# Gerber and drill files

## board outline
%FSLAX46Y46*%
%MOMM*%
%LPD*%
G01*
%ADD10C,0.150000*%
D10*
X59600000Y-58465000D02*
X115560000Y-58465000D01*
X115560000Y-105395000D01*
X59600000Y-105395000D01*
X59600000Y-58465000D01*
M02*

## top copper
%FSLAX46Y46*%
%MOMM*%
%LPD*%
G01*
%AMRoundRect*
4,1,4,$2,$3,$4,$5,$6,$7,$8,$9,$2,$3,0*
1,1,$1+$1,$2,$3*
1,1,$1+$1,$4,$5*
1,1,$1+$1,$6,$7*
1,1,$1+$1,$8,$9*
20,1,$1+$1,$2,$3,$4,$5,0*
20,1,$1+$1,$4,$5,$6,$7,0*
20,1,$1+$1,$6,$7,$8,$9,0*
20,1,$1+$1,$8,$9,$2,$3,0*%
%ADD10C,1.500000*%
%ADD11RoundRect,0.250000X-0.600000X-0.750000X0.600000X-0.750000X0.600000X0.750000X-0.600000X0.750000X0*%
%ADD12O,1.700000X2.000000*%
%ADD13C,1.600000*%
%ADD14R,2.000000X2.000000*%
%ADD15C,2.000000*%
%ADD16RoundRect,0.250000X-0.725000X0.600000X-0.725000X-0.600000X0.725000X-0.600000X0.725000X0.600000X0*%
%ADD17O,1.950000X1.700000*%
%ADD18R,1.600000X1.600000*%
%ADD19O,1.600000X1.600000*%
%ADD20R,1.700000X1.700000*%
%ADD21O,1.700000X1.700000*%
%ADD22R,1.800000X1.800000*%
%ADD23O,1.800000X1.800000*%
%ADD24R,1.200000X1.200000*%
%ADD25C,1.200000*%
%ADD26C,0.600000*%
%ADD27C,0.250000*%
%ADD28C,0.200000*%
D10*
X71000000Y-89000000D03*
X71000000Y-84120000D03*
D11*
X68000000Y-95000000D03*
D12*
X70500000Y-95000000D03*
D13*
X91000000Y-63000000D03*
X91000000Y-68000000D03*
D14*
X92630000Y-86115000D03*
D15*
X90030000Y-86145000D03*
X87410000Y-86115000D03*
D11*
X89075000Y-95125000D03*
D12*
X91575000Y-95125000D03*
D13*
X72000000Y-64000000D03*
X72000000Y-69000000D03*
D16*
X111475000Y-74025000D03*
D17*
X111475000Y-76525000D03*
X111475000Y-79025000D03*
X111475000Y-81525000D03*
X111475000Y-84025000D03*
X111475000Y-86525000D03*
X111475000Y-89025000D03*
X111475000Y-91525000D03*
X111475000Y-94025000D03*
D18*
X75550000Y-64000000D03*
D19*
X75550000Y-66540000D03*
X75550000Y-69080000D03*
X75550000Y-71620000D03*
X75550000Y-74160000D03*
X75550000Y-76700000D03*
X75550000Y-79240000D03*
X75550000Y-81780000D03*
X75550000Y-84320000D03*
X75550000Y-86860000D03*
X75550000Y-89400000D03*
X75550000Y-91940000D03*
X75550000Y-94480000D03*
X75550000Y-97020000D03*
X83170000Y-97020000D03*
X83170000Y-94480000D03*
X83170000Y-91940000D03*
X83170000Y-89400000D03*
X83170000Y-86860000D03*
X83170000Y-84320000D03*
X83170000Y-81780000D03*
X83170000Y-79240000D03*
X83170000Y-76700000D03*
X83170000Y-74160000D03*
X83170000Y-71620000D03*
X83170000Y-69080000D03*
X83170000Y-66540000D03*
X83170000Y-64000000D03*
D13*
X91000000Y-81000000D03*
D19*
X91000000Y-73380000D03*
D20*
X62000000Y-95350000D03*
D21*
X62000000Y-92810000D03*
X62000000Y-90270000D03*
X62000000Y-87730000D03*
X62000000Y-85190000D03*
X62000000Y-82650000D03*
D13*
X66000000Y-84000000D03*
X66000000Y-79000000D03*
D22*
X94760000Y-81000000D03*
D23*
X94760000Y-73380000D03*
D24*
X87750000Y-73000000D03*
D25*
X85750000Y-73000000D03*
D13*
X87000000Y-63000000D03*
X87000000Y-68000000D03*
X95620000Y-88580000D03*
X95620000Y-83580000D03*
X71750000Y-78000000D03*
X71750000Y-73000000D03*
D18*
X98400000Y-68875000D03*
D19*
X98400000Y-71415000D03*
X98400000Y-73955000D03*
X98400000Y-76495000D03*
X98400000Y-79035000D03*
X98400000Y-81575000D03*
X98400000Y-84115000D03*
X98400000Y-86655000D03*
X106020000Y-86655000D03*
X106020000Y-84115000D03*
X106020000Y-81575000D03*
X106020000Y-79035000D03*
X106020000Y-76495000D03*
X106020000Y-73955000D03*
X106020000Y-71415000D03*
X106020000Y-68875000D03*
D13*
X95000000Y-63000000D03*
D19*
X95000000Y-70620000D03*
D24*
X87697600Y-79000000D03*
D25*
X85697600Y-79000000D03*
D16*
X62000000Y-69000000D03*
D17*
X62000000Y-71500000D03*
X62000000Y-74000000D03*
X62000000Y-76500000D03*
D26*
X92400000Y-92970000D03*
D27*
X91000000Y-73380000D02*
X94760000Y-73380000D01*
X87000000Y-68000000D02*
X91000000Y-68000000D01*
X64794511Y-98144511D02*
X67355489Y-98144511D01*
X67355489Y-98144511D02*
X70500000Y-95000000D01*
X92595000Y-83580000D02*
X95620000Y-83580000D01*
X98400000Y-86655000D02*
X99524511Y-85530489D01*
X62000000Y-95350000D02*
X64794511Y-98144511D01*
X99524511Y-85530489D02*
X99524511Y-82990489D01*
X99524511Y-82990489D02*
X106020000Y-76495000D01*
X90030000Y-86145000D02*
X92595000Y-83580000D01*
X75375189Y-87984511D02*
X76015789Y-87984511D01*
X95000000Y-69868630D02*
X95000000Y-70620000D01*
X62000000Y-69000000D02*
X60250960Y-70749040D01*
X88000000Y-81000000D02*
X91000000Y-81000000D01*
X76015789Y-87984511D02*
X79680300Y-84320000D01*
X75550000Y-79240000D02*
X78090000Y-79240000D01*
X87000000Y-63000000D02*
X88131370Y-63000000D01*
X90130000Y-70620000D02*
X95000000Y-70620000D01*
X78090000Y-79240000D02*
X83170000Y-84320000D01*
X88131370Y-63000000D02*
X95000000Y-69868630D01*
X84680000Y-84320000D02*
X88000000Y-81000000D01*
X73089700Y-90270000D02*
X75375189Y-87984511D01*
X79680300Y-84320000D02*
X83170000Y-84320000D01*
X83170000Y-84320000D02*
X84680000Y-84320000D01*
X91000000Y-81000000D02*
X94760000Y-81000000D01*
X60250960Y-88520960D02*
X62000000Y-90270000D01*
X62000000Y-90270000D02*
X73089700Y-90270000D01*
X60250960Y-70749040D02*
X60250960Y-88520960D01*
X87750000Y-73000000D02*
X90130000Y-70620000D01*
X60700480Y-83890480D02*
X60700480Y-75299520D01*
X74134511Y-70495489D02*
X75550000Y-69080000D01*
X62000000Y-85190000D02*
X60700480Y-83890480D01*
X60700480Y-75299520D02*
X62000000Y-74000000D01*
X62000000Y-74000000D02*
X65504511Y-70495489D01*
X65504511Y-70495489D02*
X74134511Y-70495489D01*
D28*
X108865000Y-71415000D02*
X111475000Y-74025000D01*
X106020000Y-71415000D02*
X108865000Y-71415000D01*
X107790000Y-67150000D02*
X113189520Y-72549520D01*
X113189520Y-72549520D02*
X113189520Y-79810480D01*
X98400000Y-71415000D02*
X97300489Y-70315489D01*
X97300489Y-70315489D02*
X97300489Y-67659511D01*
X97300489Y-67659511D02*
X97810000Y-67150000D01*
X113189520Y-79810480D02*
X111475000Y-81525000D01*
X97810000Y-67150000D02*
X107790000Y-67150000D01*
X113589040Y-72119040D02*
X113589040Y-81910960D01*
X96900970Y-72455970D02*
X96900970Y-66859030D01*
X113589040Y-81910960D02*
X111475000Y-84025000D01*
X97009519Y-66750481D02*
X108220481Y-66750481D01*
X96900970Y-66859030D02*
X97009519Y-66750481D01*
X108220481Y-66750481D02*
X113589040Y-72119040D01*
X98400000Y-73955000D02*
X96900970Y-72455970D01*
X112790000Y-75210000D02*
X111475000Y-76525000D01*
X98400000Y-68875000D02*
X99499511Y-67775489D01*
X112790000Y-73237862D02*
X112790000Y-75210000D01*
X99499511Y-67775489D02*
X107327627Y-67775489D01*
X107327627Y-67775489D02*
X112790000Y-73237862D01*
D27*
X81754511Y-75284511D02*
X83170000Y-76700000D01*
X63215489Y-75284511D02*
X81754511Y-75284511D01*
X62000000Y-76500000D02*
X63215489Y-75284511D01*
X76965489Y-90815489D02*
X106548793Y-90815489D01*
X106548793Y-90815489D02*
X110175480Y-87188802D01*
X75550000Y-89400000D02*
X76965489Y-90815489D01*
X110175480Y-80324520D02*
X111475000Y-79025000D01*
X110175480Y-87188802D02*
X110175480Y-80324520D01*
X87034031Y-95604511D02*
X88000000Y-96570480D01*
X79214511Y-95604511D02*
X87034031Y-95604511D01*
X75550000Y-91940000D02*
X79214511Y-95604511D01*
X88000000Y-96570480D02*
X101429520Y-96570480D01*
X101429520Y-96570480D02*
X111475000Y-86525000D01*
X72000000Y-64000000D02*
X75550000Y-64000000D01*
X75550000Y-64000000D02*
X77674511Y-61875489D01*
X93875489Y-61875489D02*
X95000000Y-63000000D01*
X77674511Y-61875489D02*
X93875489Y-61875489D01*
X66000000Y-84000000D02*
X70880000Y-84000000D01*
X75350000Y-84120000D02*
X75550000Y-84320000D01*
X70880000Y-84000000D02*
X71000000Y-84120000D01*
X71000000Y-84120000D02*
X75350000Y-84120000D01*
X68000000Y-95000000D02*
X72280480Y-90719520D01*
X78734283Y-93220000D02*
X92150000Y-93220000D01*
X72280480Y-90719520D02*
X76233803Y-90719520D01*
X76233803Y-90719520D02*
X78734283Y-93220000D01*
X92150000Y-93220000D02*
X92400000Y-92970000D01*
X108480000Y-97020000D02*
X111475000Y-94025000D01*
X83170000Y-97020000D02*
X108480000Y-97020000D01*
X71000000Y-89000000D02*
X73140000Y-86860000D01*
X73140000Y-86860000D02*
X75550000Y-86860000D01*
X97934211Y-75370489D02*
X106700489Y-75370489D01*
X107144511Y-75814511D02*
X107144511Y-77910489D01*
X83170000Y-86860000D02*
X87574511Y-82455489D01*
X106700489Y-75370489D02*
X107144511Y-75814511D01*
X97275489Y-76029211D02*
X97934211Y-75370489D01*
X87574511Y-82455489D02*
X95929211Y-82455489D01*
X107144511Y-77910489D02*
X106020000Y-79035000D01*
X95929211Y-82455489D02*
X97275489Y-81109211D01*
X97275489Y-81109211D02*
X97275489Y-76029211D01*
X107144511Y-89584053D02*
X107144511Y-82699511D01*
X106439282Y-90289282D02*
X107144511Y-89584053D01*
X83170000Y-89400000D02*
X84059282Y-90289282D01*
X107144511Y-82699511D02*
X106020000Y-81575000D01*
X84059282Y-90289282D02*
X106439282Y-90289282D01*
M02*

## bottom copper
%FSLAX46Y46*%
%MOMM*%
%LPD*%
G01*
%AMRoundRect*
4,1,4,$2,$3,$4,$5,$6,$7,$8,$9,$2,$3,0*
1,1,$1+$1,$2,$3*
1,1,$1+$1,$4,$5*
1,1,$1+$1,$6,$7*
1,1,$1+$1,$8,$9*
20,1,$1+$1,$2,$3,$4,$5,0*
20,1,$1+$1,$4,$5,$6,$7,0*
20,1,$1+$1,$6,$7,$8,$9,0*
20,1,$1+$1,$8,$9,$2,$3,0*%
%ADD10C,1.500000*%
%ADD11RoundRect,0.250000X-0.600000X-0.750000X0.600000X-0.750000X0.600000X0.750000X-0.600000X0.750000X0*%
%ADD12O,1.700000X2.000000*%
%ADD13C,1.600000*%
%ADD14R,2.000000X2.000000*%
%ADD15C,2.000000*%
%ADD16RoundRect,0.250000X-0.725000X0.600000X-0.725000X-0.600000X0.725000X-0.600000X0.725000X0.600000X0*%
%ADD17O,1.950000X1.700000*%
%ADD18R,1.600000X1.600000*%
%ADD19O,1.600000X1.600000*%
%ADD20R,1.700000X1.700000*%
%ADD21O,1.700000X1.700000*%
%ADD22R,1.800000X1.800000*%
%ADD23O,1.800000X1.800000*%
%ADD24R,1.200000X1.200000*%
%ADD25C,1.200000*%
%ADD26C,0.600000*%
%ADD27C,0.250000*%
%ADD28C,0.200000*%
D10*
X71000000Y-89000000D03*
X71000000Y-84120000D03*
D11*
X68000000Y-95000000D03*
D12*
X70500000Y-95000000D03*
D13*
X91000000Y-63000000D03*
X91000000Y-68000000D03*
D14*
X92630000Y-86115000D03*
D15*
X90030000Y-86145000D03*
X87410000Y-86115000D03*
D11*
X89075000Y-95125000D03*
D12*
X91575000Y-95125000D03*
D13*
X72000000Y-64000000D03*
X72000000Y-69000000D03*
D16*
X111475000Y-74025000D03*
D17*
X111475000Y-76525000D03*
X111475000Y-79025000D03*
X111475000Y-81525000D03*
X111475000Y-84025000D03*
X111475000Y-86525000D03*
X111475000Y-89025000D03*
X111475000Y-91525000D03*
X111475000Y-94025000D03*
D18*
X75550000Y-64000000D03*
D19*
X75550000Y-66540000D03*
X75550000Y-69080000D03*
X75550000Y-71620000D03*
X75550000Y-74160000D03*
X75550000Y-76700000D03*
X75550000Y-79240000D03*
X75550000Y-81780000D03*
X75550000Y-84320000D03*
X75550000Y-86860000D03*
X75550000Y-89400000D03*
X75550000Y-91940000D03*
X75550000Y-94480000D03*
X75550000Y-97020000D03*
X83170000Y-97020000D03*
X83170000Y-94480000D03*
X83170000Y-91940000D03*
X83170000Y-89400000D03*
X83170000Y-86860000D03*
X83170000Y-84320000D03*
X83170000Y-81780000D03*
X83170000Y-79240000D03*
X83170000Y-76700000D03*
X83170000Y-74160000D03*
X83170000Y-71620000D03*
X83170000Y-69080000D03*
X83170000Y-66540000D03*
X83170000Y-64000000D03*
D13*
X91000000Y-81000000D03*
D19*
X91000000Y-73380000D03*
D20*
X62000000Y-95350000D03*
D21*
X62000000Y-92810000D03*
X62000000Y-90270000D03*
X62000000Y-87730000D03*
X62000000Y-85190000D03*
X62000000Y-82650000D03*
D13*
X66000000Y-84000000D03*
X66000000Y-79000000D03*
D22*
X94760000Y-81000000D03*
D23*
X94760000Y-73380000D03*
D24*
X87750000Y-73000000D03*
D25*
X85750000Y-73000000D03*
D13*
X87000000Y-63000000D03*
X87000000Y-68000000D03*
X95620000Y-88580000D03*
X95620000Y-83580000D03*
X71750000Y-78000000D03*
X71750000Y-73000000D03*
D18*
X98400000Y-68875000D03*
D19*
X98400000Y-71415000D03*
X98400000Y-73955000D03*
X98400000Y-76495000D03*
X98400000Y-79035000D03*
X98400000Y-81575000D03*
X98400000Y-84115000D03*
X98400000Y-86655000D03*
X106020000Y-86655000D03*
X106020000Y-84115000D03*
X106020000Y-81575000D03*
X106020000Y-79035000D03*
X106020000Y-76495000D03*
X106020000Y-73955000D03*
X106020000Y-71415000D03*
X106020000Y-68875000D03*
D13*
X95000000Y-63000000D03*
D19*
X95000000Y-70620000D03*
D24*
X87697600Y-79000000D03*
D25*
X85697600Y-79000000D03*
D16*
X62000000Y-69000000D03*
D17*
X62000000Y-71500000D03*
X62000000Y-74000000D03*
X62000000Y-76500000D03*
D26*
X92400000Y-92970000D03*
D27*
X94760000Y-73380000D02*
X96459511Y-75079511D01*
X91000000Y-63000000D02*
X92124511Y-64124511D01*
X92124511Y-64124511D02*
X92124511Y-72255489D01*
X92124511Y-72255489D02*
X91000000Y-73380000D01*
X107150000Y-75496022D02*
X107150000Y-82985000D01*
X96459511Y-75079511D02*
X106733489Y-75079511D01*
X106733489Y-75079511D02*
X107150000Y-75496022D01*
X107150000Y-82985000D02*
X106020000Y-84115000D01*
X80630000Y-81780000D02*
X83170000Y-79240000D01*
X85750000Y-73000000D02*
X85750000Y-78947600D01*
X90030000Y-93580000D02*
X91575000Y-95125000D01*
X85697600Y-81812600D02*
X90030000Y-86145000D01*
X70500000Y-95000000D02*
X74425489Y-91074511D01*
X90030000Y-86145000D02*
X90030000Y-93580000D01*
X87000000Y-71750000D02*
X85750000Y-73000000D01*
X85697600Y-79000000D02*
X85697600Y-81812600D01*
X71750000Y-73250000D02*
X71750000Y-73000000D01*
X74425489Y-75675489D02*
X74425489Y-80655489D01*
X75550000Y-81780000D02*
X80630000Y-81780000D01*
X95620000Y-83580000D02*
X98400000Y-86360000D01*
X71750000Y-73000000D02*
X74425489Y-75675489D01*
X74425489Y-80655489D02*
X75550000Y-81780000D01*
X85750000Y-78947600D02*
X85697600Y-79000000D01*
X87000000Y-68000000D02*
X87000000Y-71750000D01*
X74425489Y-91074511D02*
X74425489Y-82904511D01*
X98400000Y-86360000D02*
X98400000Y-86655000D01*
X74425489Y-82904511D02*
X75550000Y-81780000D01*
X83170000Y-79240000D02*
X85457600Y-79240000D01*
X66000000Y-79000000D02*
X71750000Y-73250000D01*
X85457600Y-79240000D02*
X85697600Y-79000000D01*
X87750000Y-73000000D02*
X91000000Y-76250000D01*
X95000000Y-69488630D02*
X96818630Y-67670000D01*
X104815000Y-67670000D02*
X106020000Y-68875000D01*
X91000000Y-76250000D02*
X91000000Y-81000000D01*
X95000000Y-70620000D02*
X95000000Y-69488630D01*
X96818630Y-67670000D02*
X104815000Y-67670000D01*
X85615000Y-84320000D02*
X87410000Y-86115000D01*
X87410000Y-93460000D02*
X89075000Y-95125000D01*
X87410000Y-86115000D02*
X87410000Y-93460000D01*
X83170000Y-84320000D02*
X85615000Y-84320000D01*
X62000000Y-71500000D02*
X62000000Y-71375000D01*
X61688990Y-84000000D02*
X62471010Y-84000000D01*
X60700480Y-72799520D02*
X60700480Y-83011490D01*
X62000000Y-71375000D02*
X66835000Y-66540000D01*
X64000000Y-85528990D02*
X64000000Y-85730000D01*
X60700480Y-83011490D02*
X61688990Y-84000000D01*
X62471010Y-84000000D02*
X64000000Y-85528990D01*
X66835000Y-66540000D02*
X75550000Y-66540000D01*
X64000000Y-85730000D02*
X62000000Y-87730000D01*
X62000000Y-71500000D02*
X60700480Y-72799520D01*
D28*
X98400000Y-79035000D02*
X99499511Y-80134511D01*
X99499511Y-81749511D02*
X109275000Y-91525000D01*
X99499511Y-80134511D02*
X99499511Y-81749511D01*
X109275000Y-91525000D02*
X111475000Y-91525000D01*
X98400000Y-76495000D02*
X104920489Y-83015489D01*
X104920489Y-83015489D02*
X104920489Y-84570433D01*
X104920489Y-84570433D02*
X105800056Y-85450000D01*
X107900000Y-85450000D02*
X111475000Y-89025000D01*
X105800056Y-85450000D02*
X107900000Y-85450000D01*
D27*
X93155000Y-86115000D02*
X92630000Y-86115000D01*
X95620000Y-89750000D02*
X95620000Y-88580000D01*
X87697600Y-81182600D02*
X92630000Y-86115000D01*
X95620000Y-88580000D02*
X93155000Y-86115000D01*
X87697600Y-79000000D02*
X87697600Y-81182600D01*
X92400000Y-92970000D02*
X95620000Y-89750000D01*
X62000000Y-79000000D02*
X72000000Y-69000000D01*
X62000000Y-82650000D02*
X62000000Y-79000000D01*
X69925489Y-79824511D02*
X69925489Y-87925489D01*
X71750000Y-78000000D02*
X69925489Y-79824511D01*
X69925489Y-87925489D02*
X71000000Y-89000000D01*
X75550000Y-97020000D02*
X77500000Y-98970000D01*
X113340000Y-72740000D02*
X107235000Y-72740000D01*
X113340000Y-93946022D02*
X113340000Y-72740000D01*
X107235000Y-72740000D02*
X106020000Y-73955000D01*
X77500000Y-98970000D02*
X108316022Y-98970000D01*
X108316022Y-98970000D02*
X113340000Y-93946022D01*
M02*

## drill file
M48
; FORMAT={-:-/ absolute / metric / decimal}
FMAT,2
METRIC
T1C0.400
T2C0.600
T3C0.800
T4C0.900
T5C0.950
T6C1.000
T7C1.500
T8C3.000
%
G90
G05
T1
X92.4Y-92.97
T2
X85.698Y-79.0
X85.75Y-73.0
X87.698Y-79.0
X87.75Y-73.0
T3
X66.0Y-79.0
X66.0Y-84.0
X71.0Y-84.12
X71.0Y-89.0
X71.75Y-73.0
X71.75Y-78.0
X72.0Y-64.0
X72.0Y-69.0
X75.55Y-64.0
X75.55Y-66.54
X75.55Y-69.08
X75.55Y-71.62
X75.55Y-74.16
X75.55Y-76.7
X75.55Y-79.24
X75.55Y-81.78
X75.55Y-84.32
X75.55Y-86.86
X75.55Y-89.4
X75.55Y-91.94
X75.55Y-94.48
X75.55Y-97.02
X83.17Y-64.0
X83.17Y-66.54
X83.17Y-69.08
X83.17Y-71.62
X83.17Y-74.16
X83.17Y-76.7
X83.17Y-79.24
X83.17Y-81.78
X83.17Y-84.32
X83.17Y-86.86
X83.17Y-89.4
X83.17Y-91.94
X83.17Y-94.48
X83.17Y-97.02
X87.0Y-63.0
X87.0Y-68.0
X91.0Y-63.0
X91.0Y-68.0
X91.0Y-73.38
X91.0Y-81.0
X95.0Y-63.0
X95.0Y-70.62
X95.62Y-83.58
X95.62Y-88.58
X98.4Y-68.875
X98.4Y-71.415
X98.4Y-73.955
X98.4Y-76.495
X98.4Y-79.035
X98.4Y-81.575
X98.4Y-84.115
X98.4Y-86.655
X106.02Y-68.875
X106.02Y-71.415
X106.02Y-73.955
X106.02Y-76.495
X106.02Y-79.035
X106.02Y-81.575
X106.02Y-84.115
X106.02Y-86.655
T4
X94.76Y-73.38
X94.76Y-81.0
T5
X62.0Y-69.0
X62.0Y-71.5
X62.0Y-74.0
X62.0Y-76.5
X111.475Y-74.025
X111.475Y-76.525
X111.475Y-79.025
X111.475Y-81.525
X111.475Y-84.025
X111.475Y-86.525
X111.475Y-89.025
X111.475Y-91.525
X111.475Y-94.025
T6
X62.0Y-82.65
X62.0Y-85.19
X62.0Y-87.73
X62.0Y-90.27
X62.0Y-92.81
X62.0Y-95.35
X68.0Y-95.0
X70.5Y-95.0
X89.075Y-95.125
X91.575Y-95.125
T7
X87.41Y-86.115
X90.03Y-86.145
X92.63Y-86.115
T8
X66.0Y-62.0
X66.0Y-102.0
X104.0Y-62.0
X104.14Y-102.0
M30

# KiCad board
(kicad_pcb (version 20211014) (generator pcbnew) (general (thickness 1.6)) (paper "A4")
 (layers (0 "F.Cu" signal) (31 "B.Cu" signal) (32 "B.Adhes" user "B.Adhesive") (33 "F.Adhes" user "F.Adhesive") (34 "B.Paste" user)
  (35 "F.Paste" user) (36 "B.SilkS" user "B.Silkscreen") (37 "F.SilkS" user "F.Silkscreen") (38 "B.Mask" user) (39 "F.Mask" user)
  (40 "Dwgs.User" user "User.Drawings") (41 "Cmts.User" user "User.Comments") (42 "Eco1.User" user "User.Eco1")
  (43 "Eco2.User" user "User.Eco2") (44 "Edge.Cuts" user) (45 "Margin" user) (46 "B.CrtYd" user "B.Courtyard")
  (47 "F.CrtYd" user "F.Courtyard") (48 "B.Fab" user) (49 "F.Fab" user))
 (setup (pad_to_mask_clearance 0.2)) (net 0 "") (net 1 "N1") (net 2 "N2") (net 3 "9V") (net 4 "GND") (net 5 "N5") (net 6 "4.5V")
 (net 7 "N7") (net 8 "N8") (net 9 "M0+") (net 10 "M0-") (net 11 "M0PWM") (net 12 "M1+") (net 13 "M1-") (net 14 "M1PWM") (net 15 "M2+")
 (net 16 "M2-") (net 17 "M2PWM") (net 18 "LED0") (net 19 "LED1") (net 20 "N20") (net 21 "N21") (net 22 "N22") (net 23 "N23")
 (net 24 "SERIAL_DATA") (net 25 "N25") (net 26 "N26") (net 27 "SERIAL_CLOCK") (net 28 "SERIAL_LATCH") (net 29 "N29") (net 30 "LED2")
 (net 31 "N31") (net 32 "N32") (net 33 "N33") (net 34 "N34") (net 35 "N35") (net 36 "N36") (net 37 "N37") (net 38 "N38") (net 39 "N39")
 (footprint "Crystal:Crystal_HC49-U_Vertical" (layer "F.Cu") (at 71 89 90)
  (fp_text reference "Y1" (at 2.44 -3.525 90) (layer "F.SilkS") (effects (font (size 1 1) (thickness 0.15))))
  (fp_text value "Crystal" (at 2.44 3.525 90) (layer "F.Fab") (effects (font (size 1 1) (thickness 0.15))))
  (pad "1" thru_hole circle (at 0 0 90) (size 1.5 1.5) (drill 0.8) (layers *.Cu *.Mask) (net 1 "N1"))
  (pad "2" thru_hole circle (at 4.88 0 90) (size 1.5 1.5) (drill 0.8) (layers *.Cu *.Mask) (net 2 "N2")))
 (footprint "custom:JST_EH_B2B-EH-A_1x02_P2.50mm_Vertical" (layer "F.Cu") (at 68 95)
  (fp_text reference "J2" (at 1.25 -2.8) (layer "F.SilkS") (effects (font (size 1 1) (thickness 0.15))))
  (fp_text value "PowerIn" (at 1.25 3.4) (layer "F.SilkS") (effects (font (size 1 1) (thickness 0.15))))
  (pad "1" thru_hole roundrect locked (at 0 0) (size 1.7 2) (drill 1) (layers *.Cu *.Mask) (roundrect_rratio 0.147059) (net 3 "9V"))
  (pad "2" thru_hole oval locked (at 2.5 0) (size 1.7 2) (drill 1) (layers *.Cu *.Mask) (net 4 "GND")))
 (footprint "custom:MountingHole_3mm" (layer "F.Cu") (at 104.14 102)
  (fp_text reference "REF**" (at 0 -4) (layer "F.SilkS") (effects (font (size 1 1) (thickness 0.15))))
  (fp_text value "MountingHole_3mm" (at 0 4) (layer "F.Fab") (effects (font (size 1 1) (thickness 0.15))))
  (pad "" np_thru_hole circle locked (at 0 0) (size 3 3) (drill 3) (layers *.Cu *.Mask)))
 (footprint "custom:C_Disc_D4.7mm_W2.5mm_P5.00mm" (layer "F.Cu") (at 91 63 -90)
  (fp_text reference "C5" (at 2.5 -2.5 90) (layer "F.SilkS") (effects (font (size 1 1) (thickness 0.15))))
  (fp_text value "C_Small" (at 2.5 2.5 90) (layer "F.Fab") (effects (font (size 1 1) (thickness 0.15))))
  (pad "1" thru_hole circle locked (at 0 0 270) (size 1.6 1.6) (drill 0.8) (layers *.Cu *.Mask) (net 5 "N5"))
  (pad "2" thru_hole circle locked (at 5 0 270) (size 1.6 1.6) (drill 0.8) (layers *.Cu *.Mask) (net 4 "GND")))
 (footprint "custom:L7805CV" (layer "F.Cu") (at 93.64 87.035 180)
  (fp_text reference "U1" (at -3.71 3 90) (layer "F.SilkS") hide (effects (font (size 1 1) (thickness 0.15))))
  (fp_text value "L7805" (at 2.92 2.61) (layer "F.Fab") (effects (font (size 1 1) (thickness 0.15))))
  (pad "1" thru_hole rect (at 1.01 0.92 180) (size 2 2) (drill 1.5) (layers *.Cu *.Mask) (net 3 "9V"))
  (pad "2" thru_hole circle (at 3.61 0.89 180) (size 2 2) (drill 1.5) (layers *.Cu *.Mask) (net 4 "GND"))
  (pad "3" thru_hole circle (at 6.23 0.92 180) (size 2 2) (drill 1.5) (layers *.Cu *.Mask) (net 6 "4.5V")))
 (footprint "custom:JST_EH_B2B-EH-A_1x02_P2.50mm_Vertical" (layer "F.Cu") (at 89.075 95.125)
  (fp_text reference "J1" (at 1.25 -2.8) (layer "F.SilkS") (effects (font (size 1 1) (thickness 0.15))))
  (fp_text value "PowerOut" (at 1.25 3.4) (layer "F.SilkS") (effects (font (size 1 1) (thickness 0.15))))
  (pad "1" thru_hole roundrect locked (at 0 0) (size 1.7 2) (drill 1) (layers *.Cu *.Mask) (roundrect_rratio 0.147059) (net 6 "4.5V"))
  (pad "2" thru_hole oval locked (at 2.5 0) (size 1.7 2) (drill 1) (layers *.Cu *.Mask) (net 4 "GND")))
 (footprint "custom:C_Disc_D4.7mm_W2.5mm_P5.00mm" (layer "F.Cu") (at 72 64 -90)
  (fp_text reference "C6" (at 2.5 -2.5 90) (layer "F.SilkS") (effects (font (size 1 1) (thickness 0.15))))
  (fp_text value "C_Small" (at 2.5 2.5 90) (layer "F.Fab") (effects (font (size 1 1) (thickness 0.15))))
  (pad "1" thru_hole circle locked (at 0 0 270) (size 1.6 1.6) (drill 0.8) (layers *.Cu *.Mask) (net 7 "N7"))
  (pad "2" thru_hole circle locked (at 5 0 270) (size 1.6 1.6) (drill 0.8) (layers *.Cu *.Mask) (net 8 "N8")))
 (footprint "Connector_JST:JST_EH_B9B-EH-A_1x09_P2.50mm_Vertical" (layer "F.Cu") (at 111.475 74.025 -90)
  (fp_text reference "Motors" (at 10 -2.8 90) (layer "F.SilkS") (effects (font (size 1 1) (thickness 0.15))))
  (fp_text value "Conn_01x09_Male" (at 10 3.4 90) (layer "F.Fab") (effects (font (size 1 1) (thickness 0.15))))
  (pad "1" thru_hole roundrect (at 0 0 270) (size 1.7 1.95) (drill 0.95) (layers *.Cu *.Mask) (roundrect_rratio 0.147059) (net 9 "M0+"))
  (pad "2" thru_hole oval (at 2.5 0 270) (size 1.7 1.95) (drill 0.95) (layers *.Cu *.Mask) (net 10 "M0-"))
  (pad "3" thru_hole oval (at 5 0 270) (size 1.7 1.95) (drill 0.95) (layers *.Cu *.Mask) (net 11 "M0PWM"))
  (pad "4" thru_hole oval (at 7.5 0 270) (size 1.7 1.95) (drill 0.95) (layers *.Cu *.Mask) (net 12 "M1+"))
  (pad "5" thru_hole oval (at 10 0 270) (size 1.7 1.95) (drill 0.95) (layers *.Cu *.Mask) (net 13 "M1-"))
  (pad "6" thru_hole oval (at 12.5 0 270) (size 1.7 1.95) (drill 0.95) (layers *.Cu *.Mask) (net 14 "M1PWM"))
  (pad "7" thru_hole oval (at 15 0 270) (size 1.7 1.95) (drill 0.95) (layers *.Cu *.Mask) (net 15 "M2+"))
  (pad "8" thru_hole oval (at 17.5 0 270) (size 1.7 1.95) (drill 0.95) (layers *.Cu *.Mask) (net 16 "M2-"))
  (pad "9" thru_hole oval (at 20 0 270) (size 1.7 1.95) (drill 0.95) (layers *.Cu *.Mask) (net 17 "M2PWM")))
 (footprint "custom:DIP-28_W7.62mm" (layer "F.Cu") (at 75.55 64)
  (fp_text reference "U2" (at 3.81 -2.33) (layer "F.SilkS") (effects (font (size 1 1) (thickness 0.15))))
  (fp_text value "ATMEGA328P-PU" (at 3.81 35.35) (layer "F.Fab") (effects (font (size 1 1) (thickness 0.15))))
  (pad "1" thru_hole rect locked (at 0 0) (size 1.6 1.6) (drill 0.8) (layers *.Cu *.Mask) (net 7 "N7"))
  (pad "2" thru_hole oval locked (at 0 2.54) (size 1.6 1.6) (drill 0.8) (layers *.Cu *.Mask) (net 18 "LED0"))
  (pad "3" thru_hole oval locked (at 0 5.08) (size 1.6 1.6) (drill 0.8) (layers *.Cu *.Mask) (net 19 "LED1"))
  (pad "4" thru_hole oval locked (at 0 7.62) (size 1.6 1.6) (drill 0.8) (layers *.Cu *.Mask) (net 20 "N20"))
  (pad "5" thru_hole oval locked (at 0 10.16) (size 1.6 1.6) (drill 0.8) (layers *.Cu *.Mask) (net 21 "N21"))
  (pad "6" thru_hole oval locked (at 0 12.7) (size 1.6 1.6) (drill 0.8) (layers *.Cu *.Mask) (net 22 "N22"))
  (pad "7" thru_hole oval locked (at 0 15.24) (size 1.6 1.6) (drill 0.8) (layers *.Cu *.Mask) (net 6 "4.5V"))
  (pad "8" thru_hole oval locked (at 0 17.78) (size 1.6 1.6) (drill 0.8) (layers *.Cu *.Mask) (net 4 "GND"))
  (pad "9" thru_hole oval locked (at 0 20.32) (size 1.6 1.6) (drill 0.8) (layers *.Cu *.Mask) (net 2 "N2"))
  (pad "10" thru_hole oval locked (at 0 22.86) (size 1.6 1.6) (drill 0.8) (layers *.Cu *.Mask) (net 1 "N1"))
  (pad "11" thru_hole oval locked (at 0 25.4) (size 1.6 1.6) (drill 0.8) (layers *.Cu *.Mask) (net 11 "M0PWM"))
  (pad "12" thru_hole oval locked (at 0 27.94) (size 1.6 1.6) (drill 0.8) (layers *.Cu *.Mask) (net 14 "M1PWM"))
  (pad "13" thru_hole oval locked (at 0 30.48) (size 1.6 1.6) (drill 0.8) (layers *.Cu *.Mask) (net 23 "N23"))
  (pad "14" thru_hole oval locked (at 0 33.02) (size 1.6 1.6) (drill 0.8) (layers *.Cu *.Mask) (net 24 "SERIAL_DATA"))
  (pad "15" thru_hole oval locked (at 7.62 33.02) (size 1.6 1.6) (drill 0.8) (layers *.Cu *.Mask) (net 17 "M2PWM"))
  (pad "16" thru_hole oval locked (at 7.62 30.48) (size 1.6 1.6) (drill 0.8) (layers *.Cu *.Mask) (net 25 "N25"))
  (pad "17" thru_hole oval locked (at 7.62 27.94) (size 1.6 1.6) (drill 0.8) (layers *.Cu *.Mask) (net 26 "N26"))
  (pad "18" thru_hole oval locked (at 7.62 25.4) (size 1.6 1.6) (drill 0.8) (layers *.Cu *.Mask) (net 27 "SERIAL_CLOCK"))
  (pad "19" thru_hole oval locked (at 7.62 22.86) (size 1.6 1.6) (drill 0.8) (layers *.Cu *.Mask) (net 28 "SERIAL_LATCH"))
  (pad "20" thru_hole oval locked (at 7.62 20.32) (size 1.6 1.6) (drill 0.8) (layers *.Cu *.Mask) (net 6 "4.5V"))
  (pad "21" thru_hole oval locked (at 7.62 17.78) (size 1.6 1.6) (drill 0.8) (layers *.Cu *.Mask) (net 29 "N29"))
  (pad "22" thru_hole oval locked (at 7.62 15.24) (size 1.6 1.6) (drill 0.8) (layers *.Cu *.Mask) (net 4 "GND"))
  (pad "23" thru_hole oval locked (at 7.62 12.7) (size 1.6 1.6) (drill 0.8) (layers *.Cu *.Mask) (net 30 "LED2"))
  (pad "24" thru_hole oval locked (at 7.62 10.16) (size 1.6 1.6) (drill 0.8) (layers *.Cu *.Mask) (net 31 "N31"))
  (pad "25" thru_hole oval locked (at 7.62 7.62) (size 1.6 1.6) (drill 0.8) (layers *.Cu *.Mask) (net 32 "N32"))
  (pad "26" thru_hole oval locked (at 7.62 5.08) (size 1.6 1.6) (drill 0.8) (layers *.Cu *.Mask) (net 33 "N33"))
  (pad "27" thru_hole oval locked (at 7.62 2.54) (size 1.6 1.6) (drill 0.8) (layers *.Cu *.Mask) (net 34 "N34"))
  (pad "28" thru_hole oval locked (at 7.62 0) (size 1.6 1.6) (drill 0.8) (layers *.Cu *.Mask) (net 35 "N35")))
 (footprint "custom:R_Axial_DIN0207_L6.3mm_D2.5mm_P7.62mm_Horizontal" (layer "F.Cu") (at 91 81 90)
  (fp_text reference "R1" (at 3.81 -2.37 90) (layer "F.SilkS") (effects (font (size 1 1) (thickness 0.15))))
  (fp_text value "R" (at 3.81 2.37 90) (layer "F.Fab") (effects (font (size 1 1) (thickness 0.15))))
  (pad "1" thru_hole circle locked (at 0 0 90) (size 1.6 1.6) (drill 0.8) (layers *.Cu *.Mask) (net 6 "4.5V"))
  (pad "2" thru_hole oval locked (at 7.62 0 90) (size 1.6 1.6) (drill 0.8) (layers *.Cu *.Mask) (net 5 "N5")))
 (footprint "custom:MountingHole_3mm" (layer "F.Cu") (at 104 62)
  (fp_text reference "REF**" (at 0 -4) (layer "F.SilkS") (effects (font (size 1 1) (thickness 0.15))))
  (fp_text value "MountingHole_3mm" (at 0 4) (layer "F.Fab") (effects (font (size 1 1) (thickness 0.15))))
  (pad "" np_thru_hole circle locked (at 0 0) (size 3 3) (drill 3) (layers F&B.Cu *.Mask)))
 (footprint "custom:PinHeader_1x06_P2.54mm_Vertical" (layer "F.Cu") (at 62 95.35 180)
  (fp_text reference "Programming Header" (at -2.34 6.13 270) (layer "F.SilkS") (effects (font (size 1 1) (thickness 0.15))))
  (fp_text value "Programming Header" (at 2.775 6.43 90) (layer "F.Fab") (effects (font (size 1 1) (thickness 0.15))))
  (pad "1" thru_hole rect locked (at 0 0 180) (size 1.7 1.7) (drill 1) (layers *.Cu *.Mask) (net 4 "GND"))
  (pad "2" thru_hole oval locked (at 0 2.54 180) (size 1.7 1.7) (drill 1) (layers *.Cu *.Mask) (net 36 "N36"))
  (pad "3" thru_hole oval locked (at 0 5.08 180) (size 1.7 1.7) (drill 1) (layers *.Cu *.Mask) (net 6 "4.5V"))
  (pad "4" thru_hole oval locked (at 0 7.62 180) (size 1.7 1.7) (drill 1) (layers *.Cu *.Mask) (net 18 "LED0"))
  (pad "5" thru_hole oval locked (at 0 10.16 180) (size 1.7 1.7) (drill 1) (layers *.Cu *.Mask) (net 19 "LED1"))
  (pad "6" thru_hole oval locked (at 0 12.7 180) (size 1.7 1.7) (drill 1) (layers *.Cu *.Mask) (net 8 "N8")))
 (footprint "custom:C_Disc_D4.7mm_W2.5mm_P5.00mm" (layer "F.Cu") (at 66 84 90)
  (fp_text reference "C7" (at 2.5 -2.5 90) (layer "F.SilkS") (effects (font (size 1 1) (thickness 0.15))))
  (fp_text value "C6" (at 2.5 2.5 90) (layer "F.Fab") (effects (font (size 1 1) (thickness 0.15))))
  (pad "1" thru_hole circle locked (at 0 0 90) (size 1.6 1.6) (drill 0.8) (layers *.Cu *.Mask) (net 2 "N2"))
  (pad "2" thru_hole circle locked (at 5 0 90) (size 1.6 1.6) (drill 0.8) (layers *.Cu *.Mask) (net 4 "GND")))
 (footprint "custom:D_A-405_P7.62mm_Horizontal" (layer "F.Cu") (at 94.76 81 90)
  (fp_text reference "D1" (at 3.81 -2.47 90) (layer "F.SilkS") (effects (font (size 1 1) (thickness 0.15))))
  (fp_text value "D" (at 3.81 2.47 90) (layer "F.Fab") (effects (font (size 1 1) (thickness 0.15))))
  (pad "1" thru_hole rect locked (at 0 0 90) (size 1.8 1.8) (drill 0.9) (layers *.Cu *.Mask) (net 6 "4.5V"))
  (pad "2" thru_hole oval locked (at 7.62 0 90) (size 1.8 1.8) (drill 0.9) (layers *.Cu *.Mask) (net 5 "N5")))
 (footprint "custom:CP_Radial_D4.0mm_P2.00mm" (layer "F.Cu") (at 87.75 73 180)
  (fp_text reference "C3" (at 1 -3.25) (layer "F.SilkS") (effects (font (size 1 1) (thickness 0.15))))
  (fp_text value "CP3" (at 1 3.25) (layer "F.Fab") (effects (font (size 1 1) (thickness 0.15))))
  (pad "1" thru_hole rect locked (at 0 0 180) (size 1.2 1.2) (drill 0.6) (layers *.Cu *.Mask) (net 6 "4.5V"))
  (pad "2" thru_hole circle locked (at 2 0 180) (size 1.2 1.2) (drill 0.6) (layers *.Cu *.Mask) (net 4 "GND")))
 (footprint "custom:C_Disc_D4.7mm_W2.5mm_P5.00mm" (layer "F.Cu") (at 87 63 -90)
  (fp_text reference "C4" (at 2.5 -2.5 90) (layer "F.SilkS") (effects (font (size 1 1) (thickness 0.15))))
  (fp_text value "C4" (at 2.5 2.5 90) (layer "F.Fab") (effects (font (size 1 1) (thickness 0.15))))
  (pad "1" thru_hole circle locked (at 0 0 270) (size 1.6 1.6) (drill 0.8) (layers *.Cu *.Mask) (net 6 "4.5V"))
  (pad "2" thru_hole circle locked (at 5 0 270) (size 1.6 1.6) (drill 0.8) (layers *.Cu *.Mask) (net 4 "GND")))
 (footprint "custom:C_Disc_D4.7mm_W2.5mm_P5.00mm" (layer "F.Cu") (at 95.62 88.58 90)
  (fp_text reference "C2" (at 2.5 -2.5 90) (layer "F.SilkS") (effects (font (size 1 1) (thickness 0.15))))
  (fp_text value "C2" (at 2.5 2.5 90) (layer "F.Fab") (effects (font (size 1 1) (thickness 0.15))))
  (pad "1" thru_hole circle locked (at 0 0 90) (size 1.6 1.6) (drill 0.8) (layers *.Cu *.Mask) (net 3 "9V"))
  (pad "2" thru_hole circle locked (at 5 0 90) (size 1.6 1.6) (drill 0.8) (layers *.Cu *.Mask) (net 4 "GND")))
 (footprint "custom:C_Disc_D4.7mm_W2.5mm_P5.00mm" (layer "F.Cu") (at 71.75 78 90)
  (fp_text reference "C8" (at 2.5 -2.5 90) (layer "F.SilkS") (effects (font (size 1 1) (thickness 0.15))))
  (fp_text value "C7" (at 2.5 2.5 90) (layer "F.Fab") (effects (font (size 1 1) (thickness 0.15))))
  (pad "1" thru_hole circle locked (at 0 0 90) (size 1.6 1.6) (drill 0.8) (layers *.Cu *.Mask) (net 1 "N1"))
  (pad "2" thru_hole circle locked (at 5 0 90) (size 1.6 1.6) (drill 0.8) (layers *.Cu *.Mask) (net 4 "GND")))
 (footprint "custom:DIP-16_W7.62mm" (layer "F.Cu") (at 98.4 68.875)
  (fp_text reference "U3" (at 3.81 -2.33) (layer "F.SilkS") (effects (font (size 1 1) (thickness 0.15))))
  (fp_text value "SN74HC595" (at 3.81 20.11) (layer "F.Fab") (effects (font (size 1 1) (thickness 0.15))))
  (pad "1" thru_hole rect locked (at 0 0) (size 1.6 1.6) (drill 0.8) (layers *.Cu *.Mask) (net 10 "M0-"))
  (pad "2" thru_hole oval locked (at 0 2.54) (size 1.6 1.6) (drill 0.8) (layers *.Cu *.Mask) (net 12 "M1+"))
  (pad "3" thru_hole oval locked (at 0 5.08) (size 1.6 1.6) (drill 0.8) (layers *.Cu *.Mask) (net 13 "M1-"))
  (pad "4" thru_hole oval locked (at 0 7.62) (size 1.6 1.6) (drill 0.8) (layers *.Cu *.Mask) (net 15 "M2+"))
  (pad "5" thru_hole oval locked (at 0 10.16) (size 1.6 1.6) (drill 0.8) (layers *.Cu *.Mask) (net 16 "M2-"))
  (pad "6" thru_hole oval locked (at 0 12.7) (size 1.6 1.6) (drill 0.8) (layers *.Cu *.Mask) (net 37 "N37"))
  (pad "7" thru_hole oval locked (at 0 15.24) (size 1.6 1.6) (drill 0.8) (layers *.Cu *.Mask) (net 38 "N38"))
  (pad "8" thru_hole oval locked (at 0 17.78) (size 1.6 1.6) (drill 0.8) (layers *.Cu *.Mask) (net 4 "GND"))
  (pad "9" thru_hole oval locked (at 7.62 17.78) (size 1.6 1.6) (drill 0.8) (layers *.Cu *.Mask) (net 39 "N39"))
  (pad "10" thru_hole oval locked (at 7.62 15.24) (size 1.6 1.6) (drill 0.8) (layers *.Cu *.Mask) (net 5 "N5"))
  (pad "11" thru_hole oval locked (at 7.62 12.7) (size 1.6 1.6) (drill 0.8) (layers *.Cu *.Mask) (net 27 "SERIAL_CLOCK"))
  (pad "12" thru_hole oval locked (at 7.62 10.16) (size 1.6 1.6) (drill 0.8) (layers *.Cu *.Mask) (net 28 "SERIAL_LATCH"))
  (pad "13" thru_hole oval locked (at 7.62 7.62) (size 1.6 1.6) (drill 0.8) (layers *.Cu *.Mask) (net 4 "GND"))
  (pad "14" thru_hole oval locked (at 7.62 5.08) (size 1.6 1.6) (drill 0.8) (layers *.Cu *.Mask) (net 24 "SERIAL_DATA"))
  (pad "15" thru_hole oval locked (at 7.62 2.54) (size 1.6 1.6) (drill 0.8) (layers *.Cu *.Mask) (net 9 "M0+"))
  (pad "16" thru_hole oval locked (at 7.62 0) (size 1.6 1.6) (drill 0.8) (layers *.Cu *.Mask) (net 6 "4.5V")))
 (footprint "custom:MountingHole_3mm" (layer "F.Cu") (at 66 62)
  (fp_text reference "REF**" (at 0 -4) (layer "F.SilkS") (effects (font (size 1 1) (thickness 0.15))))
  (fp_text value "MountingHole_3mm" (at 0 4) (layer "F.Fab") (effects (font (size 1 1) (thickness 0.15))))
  (pad "" np_thru_hole circle locked (at 0 0) (size 3 3) (drill 3) (layers *.Cu *.Mask)))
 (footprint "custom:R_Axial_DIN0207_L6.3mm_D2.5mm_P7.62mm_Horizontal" (layer "F.Cu") (at 95 63 -90)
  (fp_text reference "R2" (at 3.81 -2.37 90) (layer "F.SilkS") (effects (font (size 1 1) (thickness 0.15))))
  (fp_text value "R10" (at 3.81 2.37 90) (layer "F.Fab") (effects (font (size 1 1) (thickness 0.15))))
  (pad "1" thru_hole circle locked (at 0 0 270) (size 1.6 1.6) (drill 0.8) (layers *.Cu *.Mask) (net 7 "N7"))
  (pad "2" thru_hole oval locked (at 7.62 0 270) (size 1.6 1.6) (drill 0.8) (layers *.Cu *.Mask) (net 6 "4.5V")))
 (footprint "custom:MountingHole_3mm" (layer "F.Cu") (at 66 102)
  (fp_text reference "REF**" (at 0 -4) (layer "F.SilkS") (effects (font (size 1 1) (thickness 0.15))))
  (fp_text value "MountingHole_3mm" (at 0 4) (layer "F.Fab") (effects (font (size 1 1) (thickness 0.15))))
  (pad "" np_thru_hole circle locked (at 0 0) (size 3 3) (drill 3) (layers *.Cu *.Mask)))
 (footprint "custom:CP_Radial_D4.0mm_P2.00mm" (layer "F.Cu") (at 87.6976 79 180)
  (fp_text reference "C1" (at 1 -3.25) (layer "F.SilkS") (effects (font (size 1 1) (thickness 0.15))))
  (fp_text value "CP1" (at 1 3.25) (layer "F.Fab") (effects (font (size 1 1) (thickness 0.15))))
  (pad "1" thru_hole rect locked (at 0 0 180) (size 1.2 1.2) (drill 0.6) (layers *.Cu *.Mask) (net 3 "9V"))
  (pad "2" thru_hole circle locked (at 2 0 180) (size 1.2 1.2) (drill 0.6) (layers *.Cu *.Mask) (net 4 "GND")))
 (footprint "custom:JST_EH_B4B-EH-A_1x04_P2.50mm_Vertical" (layer "F.Cu") (at 62 69 -90)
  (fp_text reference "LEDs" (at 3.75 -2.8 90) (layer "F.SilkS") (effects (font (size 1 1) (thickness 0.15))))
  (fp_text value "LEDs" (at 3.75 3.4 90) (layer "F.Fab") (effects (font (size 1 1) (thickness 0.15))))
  (pad "1" thru_hole roundrect locked (at 0 0 270) (size 1.7 1.95) (drill 0.95) (layers *.Cu *.Mask) (roundrect_rratio 0.147059)
   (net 6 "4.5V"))
  (pad "2" thru_hole oval locked (at 2.5 0 270) (size 1.7 1.95) (drill 0.95) (layers *.Cu *.Mask) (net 18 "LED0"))
  (pad "3" thru_hole oval locked (at 5 0 270) (size 1.7 1.95) (drill 0.95) (layers *.Cu *.Mask) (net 19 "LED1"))
  (pad "4" thru_hole oval locked (at 7.5 0 270) (size 1.7 1.95) (drill 0.95) (layers *.Cu *.Mask) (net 30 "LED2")))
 (gr_rect (start 59.6 58.465) (end 115.56 105.395) (layer "Edge.Cuts") (width 0.15) (fill none))
 (segment (start 91 73.38) (end 94.76 73.38) (width 0.25) (layer "F.Cu") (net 5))
 (segment (start 94.76 73.38) (end 96.459511 75.079511) (width 0.25) (layer "B.Cu") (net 5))
 (segment (start 91 63) (end 92.124511 64.124511) (width 0.25) (layer "B.Cu") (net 5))
 (segment (start 92.124511 64.124511) (end 92.124511 72.255489) (width 0.25) (layer "B.Cu") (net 5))
 (segment (start 92.124511 72.255489) (end 91 73.38) (width 0.25) (layer "B.Cu") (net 5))
 (segment (start 107.15 75.496022) (end 107.15 82.985) (width 0.25) (layer "B.Cu") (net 5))
 (segment (start 96.459511 75.079511) (end 106.733489 75.079511) (width 0.25) (layer "B.Cu") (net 5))
 (segment (start 106.733489 75.079511) (end 107.15 75.496022) (width 0.25) (layer "B.Cu") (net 5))
 (segment (start 107.15 82.985) (end 106.02 84.115) (width 0.25) (layer "B.Cu") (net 5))
 (segment (start 87 68) (end 91 68) (width 0.25) (layer "F.Cu") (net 4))
 (segment (start 64.794511 98.144511) (end 67.355489 98.144511) (width 0.25) (layer "F.Cu") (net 4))
 (segment (start 67.355489 98.144511) (end 70.5 95) (width 0.25) (layer "F.Cu") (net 4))
 (segment (start 92.595 83.58) (end 95.62 83.58) (width 0.25) (layer "F.Cu") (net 4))
 (segment (start 98.4 86.655) (end 99.524511 85.530489) (width 0.25) (layer "F.Cu") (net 4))
 (segment (start 62 95.35) (end 64.794511 98.144511) (width 0.25) (layer "F.Cu") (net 4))
 (segment (start 99.524511 85.530489) (end 99.524511 82.990489) (width 0.25) (layer "F.Cu") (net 4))
 (segment (start 99.524511 82.990489) (end 106.02 76.495) (width 0.25) (layer "F.Cu") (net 4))
 (segment (start 90.03 86.145) (end 92.595 83.58) (width 0.25) (layer "F.Cu") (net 4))
 (segment (start 80.63 81.78) (end 83.17 79.24) (width 0.25) (layer "B.Cu") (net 4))
 (segment (start 85.75 73) (end 85.75 78.9476) (width 0.25) (layer "B.Cu") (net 4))
 (segment (start 90.03 93.58) (end 91.575 95.125) (width 0.25) (layer "B.Cu") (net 4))
 (segment (start 85.6976 81.8126) (end 90.03 86.145) (width 0.25) (layer "B.Cu") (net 4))
 (segment (start 70.5 95) (end 74.425489 91.074511) (width 0.25) (layer "B.Cu") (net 4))
 (segment (start 90.03 86.145) (end 90.03 93.58) (width 0.25) (layer "B.Cu") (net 4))
 (segment (start 87 71.75) (end 85.75 73) (width 0.25) (layer "B.Cu") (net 4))
 (segment (start 85.6976 79) (end 85.6976 81.8126) (width 0.25) (layer "B.Cu") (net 4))
 (segment (start 71.75 73.25) (end 71.75 73) (width 0.25) (layer "B.Cu") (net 4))
 (segment (start 74.425489 75.675489) (end 74.425489 80.655489) (width 0.25) (layer "B.Cu") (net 4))
 (segment (start 75.55 81.78) (end 80.63 81.78) (width 0.25) (layer "B.Cu") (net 4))
 (segment (start 95.62 83.58) (end 98.4 86.36) (width 0.25) (layer "B.Cu") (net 4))
 (segment (start 71.75 73) (end 74.425489 75.675489) (width 0.25) (layer "B.Cu") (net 4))
 (segment (start 74.425489 80.655489) (end 75.55 81.78) (width 0.25) (layer "B.Cu") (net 4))
 (segment (start 85.75 78.9476) (end 85.6976 79) (width 0.25) (layer "B.Cu") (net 4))
 (segment (start 87 68) (end 87 71.75) (width 0.25) (layer "B.Cu") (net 4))
 (segment (start 74.425489 91.074511) (end 74.425489 82.904511) (width 0.25) (layer "B.Cu") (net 4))
 (segment (start 98.4 86.36) (end 98.4 86.655) (width 0.25) (layer "B.Cu") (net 4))
 (segment (start 74.425489 82.904511) (end 75.55 81.78) (width 0.25) (layer "B.Cu") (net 4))
 (segment (start 83.17 79.24) (end 85.4576 79.24) (width 0.25) (layer "B.Cu") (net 4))
 (segment (start 66 79) (end 71.75 73.25) (width 0.25) (layer "B.Cu") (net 4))
 (segment (start 85.4576 79.24) (end 85.6976 79) (width 0.25) (layer "B.Cu") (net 4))
 (segment (start 75.375189 87.984511) (end 76.015789 87.984511) (width 0.25) (layer "F.Cu") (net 6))
 (segment (start 95 69.86863) (end 95 70.62) (width 0.25) (layer "F.Cu") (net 6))
 (segment (start 62 69) (end 60.25096 70.74904) (width 0.25) (layer "F.Cu") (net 6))
 (segment (start 88 81) (end 91 81) (width 0.25) (layer "F.Cu") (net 6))
 (segment (start 76.015789 87.984511) (end 79.6803 84.32) (width 0.25) (layer "F.Cu") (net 6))
 (segment (start 75.55 79.24) (end 78.09 79.24) (width 0.25) (layer "F.Cu") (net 6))
 (segment (start 87 63) (end 88.13137 63) (width 0.25) (layer "F.Cu") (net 6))
 (segment (start 90.13 70.62) (end 95 70.62) (width 0.25) (layer "F.Cu") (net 6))
 (segment (start 78.09 79.24) (end 83.17 84.32) (width 0.25) (layer "F.Cu") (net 6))
 (segment (start 88.13137 63) (end 95 69.86863) (width 0.25) (layer "F.Cu") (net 6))
 (segment (start 84.68 84.32) (end 88 81) (width 0.25) (layer "F.Cu") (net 6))
 (segment (start 73.0897 90.27) (end 75.375189 87.984511) (width 0.25) (layer "F.Cu") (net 6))
 (segment (start 79.6803 84.32) (end 83.17 84.32) (width 0.25) (layer "F.Cu") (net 6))
 (segment (start 83.17 84.32) (end 84.68 84.32) (width 0.25) (layer "F.Cu") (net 6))
 (segment (start 91 81) (end 94.76 81) (width 0.25) (layer "F.Cu") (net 6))
 (segment (start 60.25096 88.52096) (end 62 90.27) (width 0.25) (layer "F.Cu") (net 6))
 (segment (start 62 90.27) (end 73.0897 90.27) (width 0.25) (layer "F.Cu") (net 6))
 (segment (start 60.25096 70.74904) (end 60.25096 88.52096) (width 0.25) (layer "F.Cu") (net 6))
 (segment (start 87.75 73) (end 90.13 70.62) (width 0.25) (layer "F.Cu") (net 6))
 (segment (start 87.75 73) (end 91 76.25) (width 0.25) (layer "B.Cu") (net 6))
 (segment (start 95 69.48863) (end 96.81863 67.67) (width 0.25) (layer "B.Cu") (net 6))
 (segment (start 104.815 67.67) (end 106.02 68.875) (width 0.25) (layer "B.Cu") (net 6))
 (segment (start 91 76.25) (end 91 81) (width 0.25) (layer "B.Cu") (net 6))
 (segment (start 95 70.62) (end 95 69.48863) (width 0.25) (layer "B.Cu") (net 6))
 (segment (start 96.81863 67.67) (end 104.815 67.67) (width 0.25) (layer "B.Cu") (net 6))
 (segment (start 85.615 84.32) (end 87.41 86.115) (width 0.25) (layer "B.Cu") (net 6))
 (segment (start 87.41 93.46) (end 89.075 95.125) (width 0.25) (layer "B.Cu") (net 6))
 (segment (start 87.41 86.115) (end 87.41 93.46) (width 0.25) (layer "B.Cu") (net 6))
 (segment (start 83.17 84.32) (end 85.615 84.32) (width 0.25) (layer "B.Cu") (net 6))
 (segment (start 60.70048 83.89048) (end 60.70048 75.29952) (width 0.25) (layer "F.Cu") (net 19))
 (segment (start 74.134511 70.495489) (end 75.55 69.08) (width 0.25) (layer "F.Cu") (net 19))
 (segment (start 62 85.19) (end 60.70048 83.89048) (width 0.25) (layer "F.Cu") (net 19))
 (segment (start 60.70048 75.29952) (end 62 74) (width 0.25) (layer "F.Cu") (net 19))
 (segment (start 62 74) (end 65.504511 70.495489) (width 0.25) (layer "F.Cu") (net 19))
 (segment (start 65.504511 70.495489) (end 74.134511 70.495489) (width 0.25) (layer "F.Cu") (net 19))
 (segment (start 62 71.5) (end 62 71.375) (width 0.25) (layer "B.Cu") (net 18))
 (segment (start 61.68899 84) (end 62.47101 84) (width 0.25) (layer "B.Cu") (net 18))
 (segment (start 60.70048 72.79952) (end 60.70048 83.01149) (width 0.25) (layer "B.Cu") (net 18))
 (segment (start 62 71.375) (end 66.835 66.54) (width 0.25) (layer "B.Cu") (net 18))
 (segment (start 64 85.52899) (end 64 85.73) (width 0.25) (layer "B.Cu") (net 18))
 (segment (start 60.70048 83.01149) (end 61.68899 84) (width 0.25) (layer "B.Cu") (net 18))
 (segment (start 62.47101 84) (end 64 85.52899) (width 0.25) (layer "B.Cu") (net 18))
 (segment (start 66.835 66.54) (end 75.55 66.54) (width 0.25) (layer "B.Cu") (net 18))
 (segment (start 64 85.73) (end 62 87.73) (width 0.25) (layer "B.Cu") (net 18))
 (segment (start 62 71.5) (end 60.70048 72.79952) (width 0.25) (layer "B.Cu") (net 18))
 (segment (start 108.865 71.415) (end 111.475 74.025) (width 0.2) (layer "F.Cu") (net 9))
 (segment (start 106.02 71.415) (end 108.865 71.415) (width 0.2) (layer "F.Cu") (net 9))
 (segment (start 107.79 67.15) (end 113.18952 72.54952) (width 0.2) (layer "F.Cu") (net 12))
 (segment (start 113.18952 72.54952) (end 113.18952 79.81048) (width 0.2) (layer "F.Cu") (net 12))
 (segment (start 98.4 71.415) (end 97.300489 70.315489) (width 0.2) (layer "F.Cu") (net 12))
 (segment (start 97.300489 70.315489) (end 97.300489 67.659511) (width 0.2) (layer "F.Cu") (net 12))
 (segment (start 97.300489 67.659511) (end 97.81 67.15) (width 0.2) (layer "F.Cu") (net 12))
 (segment (start 113.18952 79.81048) (end 111.475 81.525) (width 0.2) (layer "F.Cu") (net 12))
 (segment (start 97.81 67.15) (end 107.79 67.15) (width 0.2) (layer "F.Cu") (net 12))
 (segment (start 113.58904 72.11904) (end 113.58904 81.91096) (width 0.2) (layer "F.Cu") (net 13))
 (segment (start 96.90097 72.45597) (end 96.90097 66.85903) (width 0.2) (layer "F.Cu") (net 13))
 (segment (start 113.58904 81.91096) (end 111.475 84.025) (width 0.2) (layer "F.Cu") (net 13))
 (segment (start 97.009519 66.750481) (end 108.220481 66.750481) (width 0.2) (layer "F.Cu") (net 13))
 (segment (start 96.90097 66.85903) (end 97.009519 66.750481) (width 0.2) (layer "F.Cu") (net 13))
 (segment (start 108.220481 66.750481) (end 113.58904 72.11904) (width 0.2) (layer "F.Cu") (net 13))
 (segment (start 98.4 73.955) (end 96.90097 72.45597) (width 0.2) (layer "F.Cu") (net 13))
 (segment (start 98.4 79.035) (end 99.499511 80.134511) (width 0.2) (layer "B.Cu") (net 16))
 (segment (start 99.499511 81.749511) (end 109.275 91.525) (width 0.2) (layer "B.Cu") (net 16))
 (segment (start 99.499511 80.134511) (end 99.499511 81.749511) (width 0.2) (layer "B.Cu") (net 16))
 (segment (start 109.275 91.525) (end 111.475 91.525) (width 0.2) (layer "B.Cu") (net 16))
 (segment (start 112.79 75.21) (end 111.475 76.525) (width 0.2) (layer "F.Cu") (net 10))
 (segment (start 98.4 68.875) (end 99.499511 67.775489) (width 0.2) (layer "F.Cu") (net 10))
 (segment (start 112.79 73.237862) (end 112.79 75.21) (width 0.2) (layer "F.Cu") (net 10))
 (segment (start 99.499511 67.775489) (end 107.327627 67.775489) (width 0.2) (layer "F.Cu") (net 10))
 (segment (start 107.327627 67.775489) (end 112.79 73.237862) (width 0.2) (layer "F.Cu") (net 10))
 (segment (start 98.4 76.495) (end 104.920489 83.015489) (width 0.2) (layer "B.Cu") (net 15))
 (segment (start 104.920489 83.015489) (end 104.920489 84.570433) (width 0.2) (layer "B.Cu") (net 15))
 (segment (start 104.920489 84.570433) (end 105.800056 85.45) (width 0.2) (layer "B.Cu") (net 15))
 (segment (start 107.9 85.45) (end 111.475 89.025) (width 0.2) (layer "B.Cu") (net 15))
 (segment (start 105.800056 85.45) (end 107.9 85.45) (width 0.2) (layer "B.Cu") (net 15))
 (segment (start 81.754511 75.284511) (end 83.17 76.7) (width 0.25) (layer "F.Cu") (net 30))
 (segment (start 63.215489 75.284511) (end 81.754511 75.284511) (width 0.25) (layer "F.Cu") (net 30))
 (segment (start 62 76.5) (end 63.215489 75.284511) (width 0.25) (layer "F.Cu") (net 30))
 (segment (start 76.965489 90.815489) (end 106.548793 90.815489) (width 0.25) (layer "F.Cu") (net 11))
 (segment (start 106.548793 90.815489) (end 110.17548 87.188802) (width 0.25) (layer "F.Cu") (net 11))
 (segment (start 75.55 89.4) (end 76.965489 90.815489) (width 0.25) (layer "F.Cu") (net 11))
 (segment (start 110.17548 80.32452) (end 111.475 79.025) (width 0.25) (layer "F.Cu") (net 11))
 (segment (start 110.17548 87.188802) (end 110.17548 80.32452) (width 0.25) (layer "F.Cu") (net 11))
 (segment (start 87.034031 95.604511) (end 88 96.57048) (width 0.25) (layer "F.Cu") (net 14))
 (segment (start 79.214511 95.604511) (end 87.034031 95.604511) (width 0.25) (layer "F.Cu") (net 14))
 (segment (start 75.55 91.94) (end 79.214511 95.604511) (width 0.25) (layer "F.Cu") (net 14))
 (segment (start 88 96.57048) (end 101.42952 96.57048) (width 0.25) (layer "F.Cu") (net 14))
 (segment (start 101.42952 96.57048) (end 111.475 86.525) (width 0.25) (layer "F.Cu") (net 14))
 (segment (start 72 64) (end 75.55 64) (width 0.25) (layer "F.Cu") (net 7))
 (segment (start 75.55 64) (end 77.674511 61.875489) (width 0.25) (layer "F.Cu") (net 7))
 (segment (start 93.875489 61.875489) (end 95 63) (width 0.25) (layer "F.Cu") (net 7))
 (segment (start 77.674511 61.875489) (end 93.875489 61.875489) (width 0.25) (layer "F.Cu") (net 7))
 (segment (start 66 84) (end 70.88 84) (width 0.25) (layer "F.Cu") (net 2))
 (segment (start 75.35 84.12) (end 75.55 84.32) (width 0.25) (layer "F.Cu") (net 2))
 (segment (start 70.88 84) (end 71 84.12) (width 0.25) (layer "F.Cu") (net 2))
 (segment (start 71 84.12) (end 75.35 84.12) (width 0.25) (layer "F.Cu") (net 2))
 (segment (start 68 95) (end 72.28048 90.71952) (width 0.25) (layer "F.Cu") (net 3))
 (segment (start 78.734283 93.22) (end 92.15 93.22) (width 0.25) (layer "F.Cu") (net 3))
 (segment (start 72.28048 90.71952) (end 76.233803 90.71952) (width 0.25) (layer "F.Cu") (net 3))
 (segment (start 76.233803 90.71952) (end 78.734283 93.22) (width 0.25) (layer "F.Cu") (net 3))
 (segment (start 92.15 93.22) (end 92.4 92.97) (width 0.25) (layer "F.Cu") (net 3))
 (via (at 92.4 92.97) (size 0.6) (drill 0.4) (layers "F.Cu" "B.Cu") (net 3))
 (segment (start 93.155 86.115) (end 92.63 86.115) (width 0.25) (layer "B.Cu") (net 3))
 (segment (start 95.62 89.75) (end 95.62 88.58) (width 0.25) (layer "B.Cu") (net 3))
 (segment (start 87.6976 81.1826) (end 92.63 86.115) (width 0.25) (layer "B.Cu") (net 3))
 (segment (start 95.62 88.58) (end 93.155 86.115) (width 0.25) (layer "B.Cu") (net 3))
 (segment (start 87.6976 79) (end 87.6976 81.1826) (width 0.25) (layer "B.Cu") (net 3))
 (segment (start 92.4 92.97) (end 95.62 89.75) (width 0.25) (layer "B.Cu") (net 3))
 (segment (start 108.48 97.02) (end 111.475 94.025) (width 0.25) (layer "F.Cu") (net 17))
 (segment (start 83.17 97.02) (end 108.48 97.02) (width 0.25) (layer "F.Cu") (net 17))
 (segment (start 62 79) (end 72 69) (width 0.25) (layer "B.Cu") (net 8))
 (segment (start 62 82.65) (end 62 79) (width 0.25) (layer "B.Cu") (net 8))
 (segment (start 71 89) (end 73.14 86.86) (width 0.25) (layer "F.Cu") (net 1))
 (segment (start 73.14 86.86) (end 75.55 86.86) (width 0.25) (layer "F.Cu") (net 1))
 (segment (start 69.925489 79.824511) (end 69.925489 87.925489) (width 0.25) (layer "B.Cu") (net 1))
 (segment (start 71.75 78) (end 69.925489 79.824511) (width 0.25) (layer "B.Cu") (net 1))
 (segment (start 69.925489 87.925489) (end 71 89) (width 0.25) (layer "B.Cu") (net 1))
 (segment (start 75.55 97.02) (end 77.5 98.97) (width 0.25) (layer "B.Cu") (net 24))
 (segment (start 113.34 72.74) (end 107.235 72.74) (width 0.25) (layer "B.Cu") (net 24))
 (segment (start 113.34 93.946022) (end 113.34 72.74) (width 0.25) (layer "B.Cu") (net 24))
 (segment (start 107.235 72.74) (end 106.02 73.955) (width 0.25) (layer "B.Cu") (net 24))
 (segment (start 77.5 98.97) (end 108.316022 98.97) (width 0.25) (layer "B.Cu") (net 24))
 (segment (start 108.316022 98.97) (end 113.34 93.946022) (width 0.25) (layer "B.Cu") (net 24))
 (segment (start 97.934211 75.370489) (end 106.700489 75.370489) (width 0.25) (layer "F.Cu") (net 28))
 (segment (start 107.144511 75.814511) (end 107.144511 77.910489) (width 0.25) (layer "F.Cu") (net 28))
 (segment (start 83.17 86.86) (end 87.574511 82.455489) (width 0.25) (layer "F.Cu") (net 28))
 (segment (start 106.700489 75.370489) (end 107.144511 75.814511) (width 0.25) (layer "F.Cu") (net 28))
 (segment (start 97.275489 76.029211) (end 97.934211 75.370489) (width 0.25) (layer "F.Cu") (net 28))
 (segment (start 87.574511 82.455489) (end 95.929211 82.455489) (width 0.25) (layer "F.Cu") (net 28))
 (segment (start 107.144511 77.910489) (end 106.02 79.035) (width 0.25) (layer "F.Cu") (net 28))
 (segment (start 95.929211 82.455489) (end 97.275489 81.109211) (width 0.25) (layer "F.Cu") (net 28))
 (segment (start 97.275489 81.109211) (end 97.275489 76.029211) (width 0.25) (layer "F.Cu") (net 28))
 (segment (start 107.144511 89.584053) (end 107.144511 82.699511) (width 0.25) (layer "F.Cu") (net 27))
 (segment (start 106.439282 90.289282) (end 107.144511 89.584053) (width 0.25) (layer "F.Cu") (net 27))
 (segment (start 83.17 89.4) (end 84.059282 90.289282) (width 0.25) (layer "F.Cu") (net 27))
 (segment (start 107.144511 82.699511) (end 106.02 81.575) (width 0.25) (layer "F.Cu") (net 27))
 (segment (start 84.059282 90.289282) (end 106.439282 90.289282) (width 0.25) (layer "F.Cu") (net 27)))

